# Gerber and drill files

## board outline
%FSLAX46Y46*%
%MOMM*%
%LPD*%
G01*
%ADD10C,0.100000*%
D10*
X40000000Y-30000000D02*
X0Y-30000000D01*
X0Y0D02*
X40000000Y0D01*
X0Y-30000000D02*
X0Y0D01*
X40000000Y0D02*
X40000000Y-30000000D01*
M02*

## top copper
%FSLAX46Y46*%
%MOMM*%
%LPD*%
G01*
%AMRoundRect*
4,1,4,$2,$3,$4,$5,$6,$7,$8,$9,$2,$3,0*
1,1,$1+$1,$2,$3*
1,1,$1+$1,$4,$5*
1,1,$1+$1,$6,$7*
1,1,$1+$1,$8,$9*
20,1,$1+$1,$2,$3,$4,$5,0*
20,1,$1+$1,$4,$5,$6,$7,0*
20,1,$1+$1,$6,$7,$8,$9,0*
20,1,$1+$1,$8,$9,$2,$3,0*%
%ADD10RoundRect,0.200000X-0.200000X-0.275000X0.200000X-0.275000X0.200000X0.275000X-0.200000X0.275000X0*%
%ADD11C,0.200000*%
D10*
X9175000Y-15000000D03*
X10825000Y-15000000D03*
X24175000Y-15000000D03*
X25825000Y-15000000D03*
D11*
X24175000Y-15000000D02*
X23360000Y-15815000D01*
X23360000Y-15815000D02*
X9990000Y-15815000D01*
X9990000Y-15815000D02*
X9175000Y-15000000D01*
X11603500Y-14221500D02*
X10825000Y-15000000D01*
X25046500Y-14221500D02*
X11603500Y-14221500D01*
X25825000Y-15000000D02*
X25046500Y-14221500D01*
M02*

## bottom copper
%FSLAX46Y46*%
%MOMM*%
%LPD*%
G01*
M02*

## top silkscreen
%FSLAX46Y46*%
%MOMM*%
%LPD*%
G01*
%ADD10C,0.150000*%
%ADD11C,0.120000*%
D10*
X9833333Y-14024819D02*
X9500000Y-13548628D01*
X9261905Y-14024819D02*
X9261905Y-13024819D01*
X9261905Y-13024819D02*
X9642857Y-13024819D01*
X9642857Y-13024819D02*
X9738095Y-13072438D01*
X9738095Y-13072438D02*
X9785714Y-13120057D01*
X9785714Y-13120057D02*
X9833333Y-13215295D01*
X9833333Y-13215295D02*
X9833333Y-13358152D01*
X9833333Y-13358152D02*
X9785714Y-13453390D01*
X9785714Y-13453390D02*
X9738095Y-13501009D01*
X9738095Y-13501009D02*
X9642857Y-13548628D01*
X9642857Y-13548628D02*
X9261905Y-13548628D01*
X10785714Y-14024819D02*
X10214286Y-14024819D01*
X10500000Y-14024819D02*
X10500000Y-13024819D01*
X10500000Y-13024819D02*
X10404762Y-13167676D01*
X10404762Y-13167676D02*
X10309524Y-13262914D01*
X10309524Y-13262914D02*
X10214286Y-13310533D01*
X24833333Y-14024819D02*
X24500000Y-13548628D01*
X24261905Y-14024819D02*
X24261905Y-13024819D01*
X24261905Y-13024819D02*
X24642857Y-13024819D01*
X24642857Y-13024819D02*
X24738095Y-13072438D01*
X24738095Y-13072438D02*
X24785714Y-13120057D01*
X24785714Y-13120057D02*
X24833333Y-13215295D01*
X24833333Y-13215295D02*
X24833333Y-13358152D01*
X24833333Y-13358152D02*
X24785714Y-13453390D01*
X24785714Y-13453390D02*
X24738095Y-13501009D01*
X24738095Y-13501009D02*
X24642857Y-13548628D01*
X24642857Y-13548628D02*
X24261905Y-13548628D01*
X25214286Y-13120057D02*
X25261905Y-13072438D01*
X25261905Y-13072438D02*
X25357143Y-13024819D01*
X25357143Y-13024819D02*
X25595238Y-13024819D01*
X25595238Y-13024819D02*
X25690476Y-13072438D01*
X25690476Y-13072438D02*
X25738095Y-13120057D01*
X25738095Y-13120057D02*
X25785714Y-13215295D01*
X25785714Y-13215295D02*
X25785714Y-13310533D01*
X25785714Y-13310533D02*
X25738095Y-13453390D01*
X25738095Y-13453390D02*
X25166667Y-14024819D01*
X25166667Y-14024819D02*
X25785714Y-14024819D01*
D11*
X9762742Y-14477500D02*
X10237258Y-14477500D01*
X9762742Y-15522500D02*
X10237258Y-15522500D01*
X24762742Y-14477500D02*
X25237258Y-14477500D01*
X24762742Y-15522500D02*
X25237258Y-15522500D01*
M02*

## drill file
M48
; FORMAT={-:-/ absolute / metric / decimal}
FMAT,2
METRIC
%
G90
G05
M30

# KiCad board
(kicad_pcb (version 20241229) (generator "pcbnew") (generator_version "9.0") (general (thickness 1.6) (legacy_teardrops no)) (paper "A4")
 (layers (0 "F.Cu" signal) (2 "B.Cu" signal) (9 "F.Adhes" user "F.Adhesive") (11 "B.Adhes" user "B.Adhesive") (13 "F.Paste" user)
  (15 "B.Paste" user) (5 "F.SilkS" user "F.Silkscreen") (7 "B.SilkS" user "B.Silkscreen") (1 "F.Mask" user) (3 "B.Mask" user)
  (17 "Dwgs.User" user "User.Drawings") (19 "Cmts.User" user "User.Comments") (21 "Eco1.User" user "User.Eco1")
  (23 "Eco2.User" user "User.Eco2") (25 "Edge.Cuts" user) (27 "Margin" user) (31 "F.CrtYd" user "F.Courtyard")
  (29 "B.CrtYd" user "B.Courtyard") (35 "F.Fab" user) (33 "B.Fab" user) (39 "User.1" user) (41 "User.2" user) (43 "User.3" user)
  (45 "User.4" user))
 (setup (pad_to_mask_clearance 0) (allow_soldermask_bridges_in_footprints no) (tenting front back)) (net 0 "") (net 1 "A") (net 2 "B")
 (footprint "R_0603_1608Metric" (layer "F.Cu") (at 10 15)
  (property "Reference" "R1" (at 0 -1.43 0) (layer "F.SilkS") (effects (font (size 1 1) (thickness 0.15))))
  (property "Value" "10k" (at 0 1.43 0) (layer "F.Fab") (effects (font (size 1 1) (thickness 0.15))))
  (fp_line (start -0.237258 -0.5225) (end 0.237258 -0.5225) (stroke (width 0.12) (type solid)) (layer "F.SilkS"))
  (fp_line (start -0.237258 0.5225) (end 0.237258 0.5225) (stroke (width 0.12) (type solid)) (layer "F.SilkS"))
  (pad "1" smd roundrect (at -0.825 0) (size 0.8 0.95) (layers "F.Cu" "F.Mask" "F.Paste") (roundrect_rratio 0.25) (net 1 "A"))
  (pad "2" smd roundrect (at 0.825 0) (size 0.8 0.95) (layers "F.Cu" "F.Mask" "F.Paste") (roundrect_rratio 0.25) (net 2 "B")))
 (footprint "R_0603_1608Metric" (layer "F.Cu") (at 25 15)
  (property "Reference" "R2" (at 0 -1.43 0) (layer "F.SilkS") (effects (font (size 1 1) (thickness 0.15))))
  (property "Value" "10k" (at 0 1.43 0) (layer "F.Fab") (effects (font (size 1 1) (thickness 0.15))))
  (fp_line (start -0.237258 -0.5225) (end 0.237258 -0.5225) (stroke (width 0.12) (type solid)) (layer "F.SilkS"))
  (fp_line (start -0.237258 0.5225) (end 0.237258 0.5225) (stroke (width 0.12) (type solid)) (layer "F.SilkS"))
  (pad "1" smd roundrect (at -0.825 0) (size 0.8 0.95) (layers "F.Cu" "F.Mask" "F.Paste") (roundrect_rratio 0.25) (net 1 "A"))
  (pad "2" smd roundrect (at 0.825 0) (size 0.8 0.95) (layers "F.Cu" "F.Mask" "F.Paste") (roundrect_rratio 0.25) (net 2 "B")))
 (gr_line (start 40 30) (end 0 30) (stroke (width 0.1) (type default)) (layer "Edge.Cuts"))
 (gr_line (start 0 0) (end 40 0) (stroke (width 0.1) (type default)) (layer "Edge.Cuts"))
 (gr_line (start 0 30) (end 0 0) (stroke (width 0.1) (type default)) (layer "Edge.Cuts"))
 (gr_line (start 40 0) (end 40 30) (stroke (width 0.1) (type default)) (layer "Edge.Cuts"))
 (segment (start 24.175 15) (end 23.36 15.815) (width 0.2) (layer "F.Cu") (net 1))
 (segment (start 23.36 15.815) (end 9.99 15.815) (width 0.2) (layer "F.Cu") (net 1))
 (segment (start 9.99 15.815) (end 9.175 15) (width 0.2) (layer "F.Cu") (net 1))
 (segment (start 11.6035 14.2215) (end 10.825 15) (width 0.2) (layer "F.Cu") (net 2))
 (segment (start 25.0465 14.2215) (end 11.6035 14.2215) (width 0.2) (layer "F.Cu") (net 2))
 (segment (start 25.825 15) (end 25.0465 14.2215) (width 0.2) (layer "F.Cu") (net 2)))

